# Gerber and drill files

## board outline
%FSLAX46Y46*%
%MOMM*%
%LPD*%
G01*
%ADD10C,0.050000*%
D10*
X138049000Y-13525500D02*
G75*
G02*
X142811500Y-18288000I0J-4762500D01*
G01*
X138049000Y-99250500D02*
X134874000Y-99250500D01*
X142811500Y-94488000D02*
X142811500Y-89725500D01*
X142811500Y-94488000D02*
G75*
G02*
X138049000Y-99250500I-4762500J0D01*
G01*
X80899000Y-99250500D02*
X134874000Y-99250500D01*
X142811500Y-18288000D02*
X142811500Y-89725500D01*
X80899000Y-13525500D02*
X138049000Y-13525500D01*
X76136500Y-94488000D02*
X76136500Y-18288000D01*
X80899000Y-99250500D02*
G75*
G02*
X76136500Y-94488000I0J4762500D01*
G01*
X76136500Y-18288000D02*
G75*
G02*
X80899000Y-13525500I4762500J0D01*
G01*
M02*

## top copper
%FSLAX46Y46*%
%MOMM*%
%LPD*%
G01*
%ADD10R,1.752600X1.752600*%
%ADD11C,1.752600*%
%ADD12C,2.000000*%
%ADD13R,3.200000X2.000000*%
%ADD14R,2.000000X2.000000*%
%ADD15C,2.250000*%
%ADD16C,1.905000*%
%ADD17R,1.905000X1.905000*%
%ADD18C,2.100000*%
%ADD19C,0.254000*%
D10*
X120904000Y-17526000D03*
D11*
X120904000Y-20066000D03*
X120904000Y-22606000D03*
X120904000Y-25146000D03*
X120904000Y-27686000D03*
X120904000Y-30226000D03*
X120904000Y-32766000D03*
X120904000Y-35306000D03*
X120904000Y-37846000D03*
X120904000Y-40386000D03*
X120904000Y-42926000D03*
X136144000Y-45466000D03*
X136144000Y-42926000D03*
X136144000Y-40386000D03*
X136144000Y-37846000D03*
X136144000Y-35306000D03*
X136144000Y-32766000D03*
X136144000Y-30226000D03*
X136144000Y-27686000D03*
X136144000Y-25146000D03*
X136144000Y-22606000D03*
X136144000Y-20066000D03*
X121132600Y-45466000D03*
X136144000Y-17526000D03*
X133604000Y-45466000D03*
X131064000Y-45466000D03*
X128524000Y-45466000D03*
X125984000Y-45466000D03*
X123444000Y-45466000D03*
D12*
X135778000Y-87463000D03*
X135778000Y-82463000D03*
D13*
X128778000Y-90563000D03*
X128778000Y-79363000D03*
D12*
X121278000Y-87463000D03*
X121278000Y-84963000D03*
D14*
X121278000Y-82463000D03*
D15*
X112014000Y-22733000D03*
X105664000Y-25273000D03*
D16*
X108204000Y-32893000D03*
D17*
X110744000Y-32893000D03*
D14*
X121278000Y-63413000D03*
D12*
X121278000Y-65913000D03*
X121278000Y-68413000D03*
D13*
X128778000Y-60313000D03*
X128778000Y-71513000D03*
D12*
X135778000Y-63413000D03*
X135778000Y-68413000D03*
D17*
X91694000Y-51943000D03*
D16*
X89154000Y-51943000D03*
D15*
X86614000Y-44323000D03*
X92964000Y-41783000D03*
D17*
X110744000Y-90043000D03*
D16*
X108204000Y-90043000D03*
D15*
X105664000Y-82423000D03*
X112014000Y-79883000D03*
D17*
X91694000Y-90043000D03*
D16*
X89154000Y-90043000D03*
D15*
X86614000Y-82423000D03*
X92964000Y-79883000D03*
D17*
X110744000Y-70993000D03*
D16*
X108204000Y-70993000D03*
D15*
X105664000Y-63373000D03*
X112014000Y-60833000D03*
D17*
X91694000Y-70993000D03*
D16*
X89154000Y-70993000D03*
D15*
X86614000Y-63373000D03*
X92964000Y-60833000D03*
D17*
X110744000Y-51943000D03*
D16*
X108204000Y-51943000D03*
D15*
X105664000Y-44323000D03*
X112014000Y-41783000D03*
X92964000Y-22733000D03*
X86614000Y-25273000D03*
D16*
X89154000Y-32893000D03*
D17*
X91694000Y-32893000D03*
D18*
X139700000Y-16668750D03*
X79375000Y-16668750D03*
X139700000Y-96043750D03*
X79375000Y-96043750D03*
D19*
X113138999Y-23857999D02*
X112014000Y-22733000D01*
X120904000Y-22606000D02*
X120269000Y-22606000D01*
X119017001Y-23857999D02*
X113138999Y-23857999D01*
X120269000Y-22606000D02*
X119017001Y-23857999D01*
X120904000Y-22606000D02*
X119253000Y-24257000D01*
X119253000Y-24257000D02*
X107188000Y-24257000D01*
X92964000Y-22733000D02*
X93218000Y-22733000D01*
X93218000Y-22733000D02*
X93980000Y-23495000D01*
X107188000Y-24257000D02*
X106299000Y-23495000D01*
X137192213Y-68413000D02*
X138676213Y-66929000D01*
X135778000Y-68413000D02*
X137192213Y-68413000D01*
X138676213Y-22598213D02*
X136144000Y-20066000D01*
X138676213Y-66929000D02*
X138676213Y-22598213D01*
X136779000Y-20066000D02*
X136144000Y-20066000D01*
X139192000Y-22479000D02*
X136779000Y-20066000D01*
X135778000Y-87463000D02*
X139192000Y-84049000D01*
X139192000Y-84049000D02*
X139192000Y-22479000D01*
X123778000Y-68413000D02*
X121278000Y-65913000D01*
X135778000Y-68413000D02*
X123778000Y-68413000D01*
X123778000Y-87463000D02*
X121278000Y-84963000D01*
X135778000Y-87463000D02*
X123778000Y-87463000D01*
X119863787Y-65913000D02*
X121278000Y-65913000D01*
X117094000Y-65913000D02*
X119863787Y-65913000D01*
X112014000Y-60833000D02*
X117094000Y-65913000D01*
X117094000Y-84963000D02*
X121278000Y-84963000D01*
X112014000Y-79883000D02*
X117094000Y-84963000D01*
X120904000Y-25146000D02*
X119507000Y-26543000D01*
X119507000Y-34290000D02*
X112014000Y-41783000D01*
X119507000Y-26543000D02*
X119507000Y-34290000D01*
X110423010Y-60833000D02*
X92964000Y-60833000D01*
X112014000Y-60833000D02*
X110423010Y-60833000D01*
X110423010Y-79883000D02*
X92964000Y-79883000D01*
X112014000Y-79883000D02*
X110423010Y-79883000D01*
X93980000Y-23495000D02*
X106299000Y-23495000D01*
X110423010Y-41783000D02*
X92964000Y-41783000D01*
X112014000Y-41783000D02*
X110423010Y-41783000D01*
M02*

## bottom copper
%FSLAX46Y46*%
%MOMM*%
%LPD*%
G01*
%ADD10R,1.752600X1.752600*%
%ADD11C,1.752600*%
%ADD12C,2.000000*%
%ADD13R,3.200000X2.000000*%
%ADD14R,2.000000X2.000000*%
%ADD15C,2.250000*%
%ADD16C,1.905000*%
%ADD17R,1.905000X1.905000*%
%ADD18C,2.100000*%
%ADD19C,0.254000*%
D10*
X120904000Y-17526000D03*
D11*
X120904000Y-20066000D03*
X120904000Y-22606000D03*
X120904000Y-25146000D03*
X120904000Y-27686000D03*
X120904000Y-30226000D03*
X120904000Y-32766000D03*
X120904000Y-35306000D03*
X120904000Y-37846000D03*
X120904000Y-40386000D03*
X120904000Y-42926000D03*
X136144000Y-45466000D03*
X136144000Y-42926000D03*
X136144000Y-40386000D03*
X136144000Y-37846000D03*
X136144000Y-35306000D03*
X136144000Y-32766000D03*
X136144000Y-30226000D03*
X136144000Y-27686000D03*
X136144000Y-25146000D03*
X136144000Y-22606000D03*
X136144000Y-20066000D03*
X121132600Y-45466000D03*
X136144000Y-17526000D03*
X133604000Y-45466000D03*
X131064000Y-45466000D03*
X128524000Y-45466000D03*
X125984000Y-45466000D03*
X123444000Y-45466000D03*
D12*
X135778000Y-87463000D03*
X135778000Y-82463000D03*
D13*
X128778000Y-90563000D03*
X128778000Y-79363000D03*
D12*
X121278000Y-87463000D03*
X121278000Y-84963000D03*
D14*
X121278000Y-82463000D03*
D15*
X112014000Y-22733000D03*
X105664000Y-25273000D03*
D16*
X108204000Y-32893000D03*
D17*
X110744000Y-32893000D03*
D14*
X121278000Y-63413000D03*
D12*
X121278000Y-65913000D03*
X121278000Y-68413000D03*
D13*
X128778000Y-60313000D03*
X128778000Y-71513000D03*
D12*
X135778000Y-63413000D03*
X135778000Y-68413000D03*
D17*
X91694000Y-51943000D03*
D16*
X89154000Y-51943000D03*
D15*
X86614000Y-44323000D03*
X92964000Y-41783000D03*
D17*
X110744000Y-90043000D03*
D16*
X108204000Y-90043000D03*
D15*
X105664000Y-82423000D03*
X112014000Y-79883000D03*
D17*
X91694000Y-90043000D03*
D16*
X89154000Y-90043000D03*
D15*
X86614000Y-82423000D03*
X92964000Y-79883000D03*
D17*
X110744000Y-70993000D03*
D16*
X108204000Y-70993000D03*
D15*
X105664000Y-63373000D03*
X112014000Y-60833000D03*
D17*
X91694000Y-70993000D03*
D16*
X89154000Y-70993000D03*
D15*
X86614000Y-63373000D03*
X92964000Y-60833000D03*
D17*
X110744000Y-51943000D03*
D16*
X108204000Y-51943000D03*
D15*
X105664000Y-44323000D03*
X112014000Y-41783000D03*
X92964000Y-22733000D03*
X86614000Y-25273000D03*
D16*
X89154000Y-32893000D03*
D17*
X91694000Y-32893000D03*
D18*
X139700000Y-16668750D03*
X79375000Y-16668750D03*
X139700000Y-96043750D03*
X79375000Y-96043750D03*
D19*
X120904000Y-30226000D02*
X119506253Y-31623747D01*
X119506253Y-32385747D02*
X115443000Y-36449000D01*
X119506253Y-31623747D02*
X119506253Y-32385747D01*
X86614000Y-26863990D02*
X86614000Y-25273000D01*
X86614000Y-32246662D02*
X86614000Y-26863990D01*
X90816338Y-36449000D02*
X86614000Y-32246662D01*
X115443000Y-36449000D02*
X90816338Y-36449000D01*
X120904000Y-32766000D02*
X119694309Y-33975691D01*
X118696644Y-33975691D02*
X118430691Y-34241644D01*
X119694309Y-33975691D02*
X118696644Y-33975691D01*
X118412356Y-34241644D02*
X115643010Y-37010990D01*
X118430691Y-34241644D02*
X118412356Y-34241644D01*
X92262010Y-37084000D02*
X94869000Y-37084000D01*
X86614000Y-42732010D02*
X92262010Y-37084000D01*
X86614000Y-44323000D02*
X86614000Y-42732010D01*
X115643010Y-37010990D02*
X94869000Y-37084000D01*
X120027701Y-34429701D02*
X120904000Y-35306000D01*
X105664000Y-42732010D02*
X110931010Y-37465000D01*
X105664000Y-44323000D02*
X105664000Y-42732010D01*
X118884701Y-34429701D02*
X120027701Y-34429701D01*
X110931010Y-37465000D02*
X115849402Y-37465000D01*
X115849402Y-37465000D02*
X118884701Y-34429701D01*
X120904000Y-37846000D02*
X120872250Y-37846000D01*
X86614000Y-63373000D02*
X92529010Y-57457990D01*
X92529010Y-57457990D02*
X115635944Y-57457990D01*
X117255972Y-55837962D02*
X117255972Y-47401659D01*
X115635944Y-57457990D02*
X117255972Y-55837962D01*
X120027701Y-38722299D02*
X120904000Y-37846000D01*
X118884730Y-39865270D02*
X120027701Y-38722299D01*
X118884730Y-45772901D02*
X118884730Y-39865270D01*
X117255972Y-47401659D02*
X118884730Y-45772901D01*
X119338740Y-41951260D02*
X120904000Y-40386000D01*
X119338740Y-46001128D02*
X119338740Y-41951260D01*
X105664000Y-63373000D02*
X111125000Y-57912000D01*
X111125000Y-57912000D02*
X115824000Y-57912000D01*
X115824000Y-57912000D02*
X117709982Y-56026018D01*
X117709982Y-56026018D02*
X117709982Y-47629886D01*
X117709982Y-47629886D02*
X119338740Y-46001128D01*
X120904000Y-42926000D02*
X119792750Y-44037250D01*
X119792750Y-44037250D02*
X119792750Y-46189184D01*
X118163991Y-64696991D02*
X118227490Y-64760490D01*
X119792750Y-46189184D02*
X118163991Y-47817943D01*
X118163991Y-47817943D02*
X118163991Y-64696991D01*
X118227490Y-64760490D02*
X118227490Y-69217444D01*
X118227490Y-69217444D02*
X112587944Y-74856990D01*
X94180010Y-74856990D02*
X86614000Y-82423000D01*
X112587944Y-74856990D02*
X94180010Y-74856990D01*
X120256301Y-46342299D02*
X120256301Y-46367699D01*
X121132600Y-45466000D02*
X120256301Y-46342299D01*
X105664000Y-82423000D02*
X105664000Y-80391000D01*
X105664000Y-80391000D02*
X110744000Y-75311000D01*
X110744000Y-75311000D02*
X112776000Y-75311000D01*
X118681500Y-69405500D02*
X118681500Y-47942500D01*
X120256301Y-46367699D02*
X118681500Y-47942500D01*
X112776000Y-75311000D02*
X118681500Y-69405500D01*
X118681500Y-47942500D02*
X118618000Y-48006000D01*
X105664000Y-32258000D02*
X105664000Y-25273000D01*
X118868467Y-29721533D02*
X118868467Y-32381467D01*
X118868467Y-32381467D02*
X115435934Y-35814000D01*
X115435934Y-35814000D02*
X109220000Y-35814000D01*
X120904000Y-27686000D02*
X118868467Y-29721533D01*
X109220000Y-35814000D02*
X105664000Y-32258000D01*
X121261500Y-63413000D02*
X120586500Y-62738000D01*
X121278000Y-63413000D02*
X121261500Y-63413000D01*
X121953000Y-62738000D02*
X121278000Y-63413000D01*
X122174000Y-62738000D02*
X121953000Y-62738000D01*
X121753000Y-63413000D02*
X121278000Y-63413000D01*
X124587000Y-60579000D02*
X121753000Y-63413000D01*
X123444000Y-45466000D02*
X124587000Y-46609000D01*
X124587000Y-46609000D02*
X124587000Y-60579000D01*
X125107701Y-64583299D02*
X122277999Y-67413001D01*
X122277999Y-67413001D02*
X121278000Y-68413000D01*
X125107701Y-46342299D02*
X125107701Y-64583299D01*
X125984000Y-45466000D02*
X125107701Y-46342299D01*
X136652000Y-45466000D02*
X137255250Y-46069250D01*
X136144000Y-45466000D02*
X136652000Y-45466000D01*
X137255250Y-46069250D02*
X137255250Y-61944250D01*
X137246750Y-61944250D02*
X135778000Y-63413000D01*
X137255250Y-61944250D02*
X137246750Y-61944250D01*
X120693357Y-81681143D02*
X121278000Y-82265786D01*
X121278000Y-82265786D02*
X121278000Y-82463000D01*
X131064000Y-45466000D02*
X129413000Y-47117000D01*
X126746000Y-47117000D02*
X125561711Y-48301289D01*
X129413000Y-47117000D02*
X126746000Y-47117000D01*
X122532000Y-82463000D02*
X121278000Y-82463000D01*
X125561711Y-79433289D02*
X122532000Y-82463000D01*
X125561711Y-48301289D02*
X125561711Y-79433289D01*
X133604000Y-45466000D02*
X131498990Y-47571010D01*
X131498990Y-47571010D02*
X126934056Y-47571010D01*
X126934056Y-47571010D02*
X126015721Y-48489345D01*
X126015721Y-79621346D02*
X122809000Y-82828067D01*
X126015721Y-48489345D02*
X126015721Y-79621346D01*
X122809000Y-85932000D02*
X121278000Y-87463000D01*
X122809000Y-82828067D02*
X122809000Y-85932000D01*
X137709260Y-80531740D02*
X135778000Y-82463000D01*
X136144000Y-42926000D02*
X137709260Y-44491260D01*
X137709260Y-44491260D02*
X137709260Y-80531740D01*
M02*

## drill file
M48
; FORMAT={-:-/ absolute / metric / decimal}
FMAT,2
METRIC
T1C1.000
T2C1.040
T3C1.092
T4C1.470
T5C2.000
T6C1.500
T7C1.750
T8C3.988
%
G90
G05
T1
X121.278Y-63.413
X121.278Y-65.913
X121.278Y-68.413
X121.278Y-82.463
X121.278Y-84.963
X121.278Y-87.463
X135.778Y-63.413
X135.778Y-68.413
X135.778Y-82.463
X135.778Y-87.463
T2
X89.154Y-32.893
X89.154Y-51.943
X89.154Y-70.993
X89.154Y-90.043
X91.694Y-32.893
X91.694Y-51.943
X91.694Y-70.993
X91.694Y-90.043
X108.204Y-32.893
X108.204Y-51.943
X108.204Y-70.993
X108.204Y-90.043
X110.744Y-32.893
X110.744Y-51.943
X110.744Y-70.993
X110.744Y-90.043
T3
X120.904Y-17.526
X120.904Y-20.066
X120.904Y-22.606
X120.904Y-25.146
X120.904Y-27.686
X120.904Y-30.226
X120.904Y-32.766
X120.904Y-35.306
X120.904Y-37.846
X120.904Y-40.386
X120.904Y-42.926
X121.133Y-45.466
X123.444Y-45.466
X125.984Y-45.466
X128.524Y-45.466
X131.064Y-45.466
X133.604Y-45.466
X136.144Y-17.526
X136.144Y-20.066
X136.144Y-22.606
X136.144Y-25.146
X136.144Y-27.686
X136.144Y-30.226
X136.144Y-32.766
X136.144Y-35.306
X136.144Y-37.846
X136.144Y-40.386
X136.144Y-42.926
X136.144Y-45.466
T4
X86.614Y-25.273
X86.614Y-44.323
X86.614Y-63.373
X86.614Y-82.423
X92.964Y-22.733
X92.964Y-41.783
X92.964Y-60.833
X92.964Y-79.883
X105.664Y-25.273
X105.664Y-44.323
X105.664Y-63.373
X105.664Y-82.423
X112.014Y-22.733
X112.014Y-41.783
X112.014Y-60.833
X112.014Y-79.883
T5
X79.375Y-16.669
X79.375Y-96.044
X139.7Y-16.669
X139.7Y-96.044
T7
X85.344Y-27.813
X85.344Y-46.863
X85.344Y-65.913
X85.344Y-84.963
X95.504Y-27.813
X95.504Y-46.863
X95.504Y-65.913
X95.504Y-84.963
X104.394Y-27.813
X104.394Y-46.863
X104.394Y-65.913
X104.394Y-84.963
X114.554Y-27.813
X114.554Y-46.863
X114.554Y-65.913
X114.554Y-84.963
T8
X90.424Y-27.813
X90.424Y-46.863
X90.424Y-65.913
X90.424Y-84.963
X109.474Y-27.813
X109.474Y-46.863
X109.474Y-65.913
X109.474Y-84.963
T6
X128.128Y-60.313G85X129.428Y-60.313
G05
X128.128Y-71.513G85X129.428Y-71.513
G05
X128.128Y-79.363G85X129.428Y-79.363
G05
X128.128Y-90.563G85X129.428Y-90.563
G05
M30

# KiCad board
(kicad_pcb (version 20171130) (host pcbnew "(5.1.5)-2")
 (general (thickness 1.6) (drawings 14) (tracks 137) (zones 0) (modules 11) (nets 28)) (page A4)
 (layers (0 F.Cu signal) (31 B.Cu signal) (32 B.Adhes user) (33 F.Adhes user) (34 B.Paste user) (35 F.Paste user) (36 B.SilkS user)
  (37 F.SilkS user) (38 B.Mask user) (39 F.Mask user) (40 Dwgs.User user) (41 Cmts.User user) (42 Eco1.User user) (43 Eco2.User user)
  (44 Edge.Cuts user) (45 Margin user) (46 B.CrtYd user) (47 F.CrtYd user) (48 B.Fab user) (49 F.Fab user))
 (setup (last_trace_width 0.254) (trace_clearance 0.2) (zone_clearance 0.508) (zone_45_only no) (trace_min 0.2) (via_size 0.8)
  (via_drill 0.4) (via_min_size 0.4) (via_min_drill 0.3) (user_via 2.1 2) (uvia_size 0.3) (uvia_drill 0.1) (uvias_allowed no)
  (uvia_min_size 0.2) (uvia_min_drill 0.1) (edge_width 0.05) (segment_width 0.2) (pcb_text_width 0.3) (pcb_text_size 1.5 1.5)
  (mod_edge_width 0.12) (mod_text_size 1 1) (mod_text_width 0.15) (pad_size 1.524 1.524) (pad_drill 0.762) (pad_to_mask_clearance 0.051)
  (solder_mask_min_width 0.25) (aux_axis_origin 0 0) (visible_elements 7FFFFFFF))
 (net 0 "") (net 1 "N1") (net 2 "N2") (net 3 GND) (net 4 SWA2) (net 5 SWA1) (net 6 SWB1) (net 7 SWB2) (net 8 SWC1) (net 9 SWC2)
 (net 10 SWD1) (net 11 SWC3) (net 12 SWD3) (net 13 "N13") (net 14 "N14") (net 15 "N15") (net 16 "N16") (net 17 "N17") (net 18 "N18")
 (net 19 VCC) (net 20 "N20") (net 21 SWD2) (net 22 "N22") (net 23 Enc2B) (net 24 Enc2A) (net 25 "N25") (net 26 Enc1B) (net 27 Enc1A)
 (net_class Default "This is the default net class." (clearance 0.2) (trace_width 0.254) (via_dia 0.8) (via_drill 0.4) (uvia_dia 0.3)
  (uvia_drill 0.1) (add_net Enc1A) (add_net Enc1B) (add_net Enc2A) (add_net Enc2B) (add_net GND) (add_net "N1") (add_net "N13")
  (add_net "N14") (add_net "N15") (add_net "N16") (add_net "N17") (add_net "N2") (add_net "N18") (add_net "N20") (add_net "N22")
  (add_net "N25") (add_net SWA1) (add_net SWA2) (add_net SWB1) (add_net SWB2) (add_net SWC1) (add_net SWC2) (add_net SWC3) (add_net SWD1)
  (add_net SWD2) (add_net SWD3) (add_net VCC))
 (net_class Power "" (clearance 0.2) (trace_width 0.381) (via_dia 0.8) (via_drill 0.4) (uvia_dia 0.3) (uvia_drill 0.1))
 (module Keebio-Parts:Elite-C (layer F.Cu) (at 128.524 31.496 270)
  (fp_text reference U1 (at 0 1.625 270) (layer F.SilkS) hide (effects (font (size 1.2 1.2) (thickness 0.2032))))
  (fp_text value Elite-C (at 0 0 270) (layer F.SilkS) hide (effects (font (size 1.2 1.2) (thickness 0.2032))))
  (pad 1 thru_hole rect (at -13.97 7.62 270) (size 1.7526 1.7526) (drill 1.0922) (layers *.Cu *.SilkS *.Mask) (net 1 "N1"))
  (pad 2 thru_hole circle (at -11.43 7.62 270) (size 1.7526 1.7526) (drill 1.0922) (layers *.Cu *.SilkS *.Mask) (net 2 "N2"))
  (pad 3 thru_hole circle (at -8.89 7.62 270) (size 1.7526 1.7526) (drill 1.0922) (layers *.Cu *.SilkS *.Mask) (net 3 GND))
  (pad 4 thru_hole circle (at -6.35 7.62 270) (size 1.7526 1.7526) (drill 1.0922) (layers *.Cu *.SilkS *.Mask) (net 3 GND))
  (pad 5 thru_hole circle (at -3.81 7.62 270) (size 1.7526 1.7526) (drill 1.0922) (layers *.Cu *.SilkS *.Mask) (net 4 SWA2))
  (pad 6 thru_hole circle (at -1.27 7.62 270) (size 1.7526 1.7526) (drill 1.0922) (layers *.Cu *.SilkS *.Mask) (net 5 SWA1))
  (pad 7 thru_hole circle (at 1.27 7.62 270) (size 1.7526 1.7526) (drill 1.0922) (layers *.Cu *.SilkS *.Mask) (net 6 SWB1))
  (pad 8 thru_hole circle (at 3.81 7.62 270) (size 1.7526 1.7526) (drill 1.0922) (layers *.Cu *.SilkS *.Mask) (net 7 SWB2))
  (pad 9 thru_hole circle (at 6.35 7.62 270) (size 1.7526 1.7526) (drill 1.0922) (layers *.Cu *.SilkS *.Mask) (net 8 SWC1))
  (pad 10 thru_hole circle (at 8.89 7.62 270) (size 1.7526 1.7526) (drill 1.0922) (layers *.Cu *.SilkS *.Mask) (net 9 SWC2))
  (pad 11 thru_hole circle (at 11.43 7.62 270) (size 1.7526 1.7526) (drill 1.0922) (layers *.Cu *.SilkS *.Mask) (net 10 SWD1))
  (pad 13 thru_hole circle (at 13.97 -7.62 270) (size 1.7526 1.7526) (drill 1.0922) (layers *.Cu *.SilkS *.Mask) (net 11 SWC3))
  (pad 14 thru_hole circle (at 11.43 -7.62 270) (size 1.7526 1.7526) (drill 1.0922) (layers *.Cu *.SilkS *.Mask) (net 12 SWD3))
  (pad 15 thru_hole circle (at 8.89 -7.62 270) (size 1.7526 1.7526) (drill 1.0922) (layers *.Cu *.SilkS *.Mask) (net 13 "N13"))
  (pad 16 thru_hole circle (at 6.35 -7.62 270) (size 1.7526 1.7526) (drill 1.0922) (layers *.Cu *.SilkS *.Mask) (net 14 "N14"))
  (pad 17 thru_hole circle (at 3.81 -7.62 270) (size 1.7526 1.7526) (drill 1.0922) (layers *.Cu *.SilkS *.Mask) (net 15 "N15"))
  (pad 18 thru_hole circle (at 1.27 -7.62 270) (size 1.7526 1.7526) (drill 1.0922) (layers *.Cu *.SilkS *.Mask) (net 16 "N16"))
  (pad 19 thru_hole circle (at -1.27 -7.62 270) (size 1.7526 1.7526) (drill 1.0922) (layers *.Cu *.SilkS *.Mask) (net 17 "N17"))
  (pad 20 thru_hole circle (at -3.81 -7.62 270) (size 1.7526 1.7526) (drill 1.0922) (layers *.Cu *.SilkS *.Mask) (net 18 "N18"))
  (pad 21 thru_hole circle (at -6.35 -7.62 270) (size 1.7526 1.7526) (drill 1.0922) (layers *.Cu *.SilkS *.Mask) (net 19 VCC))
  (pad 22 thru_hole circle (at -8.89 -7.62 270) (size 1.7526 1.7526) (drill 1.0922) (layers *.Cu *.SilkS *.Mask) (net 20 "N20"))
  (pad 23 thru_hole circle (at -11.43 -7.62 270) (size 1.7526 1.7526) (drill 1.0922) (layers *.Cu *.SilkS *.Mask) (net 3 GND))
  (pad 12 thru_hole circle (at 13.97 7.3914 270) (size 1.7526 1.7526) (drill 1.0922) (layers *.Cu *.SilkS *.Mask) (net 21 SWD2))
  (pad 24 thru_hole circle (at -13.97 -7.62 270) (size 1.7526 1.7526) (drill 1.0922) (layers *.Cu *.SilkS *.Mask) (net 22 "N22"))
  (pad 29 thru_hole circle (at 13.97 -5.08 270) (size 1.7526 1.7526) (drill 1.0922) (layers *.Cu *.SilkS *.Mask) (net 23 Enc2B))
  (pad 28 thru_hole circle (at 13.97 -2.54 270) (size 1.7526 1.7526) (drill 1.0922) (layers *.Cu *.SilkS *.Mask) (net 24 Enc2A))
  (pad 27 thru_hole circle (at 13.97 0 270) (size 1.7526 1.7526) (drill 1.0922) (layers *.Cu *.SilkS *.Mask) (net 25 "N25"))
  (pad 26 thru_hole circle (at 13.97 2.54 270) (size 1.7526 1.7526) (drill 1.0922) (layers *.Cu *.SilkS *.Mask) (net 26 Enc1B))
  (pad 25 thru_hole circle (at 13.97 5.08 270) (size 1.7526 1.7526) (drill 1.0922) (layers *.Cu *.SilkS *.Mask) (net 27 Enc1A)))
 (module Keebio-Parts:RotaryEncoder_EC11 (layer F.Cu) (at 128.778 84.963)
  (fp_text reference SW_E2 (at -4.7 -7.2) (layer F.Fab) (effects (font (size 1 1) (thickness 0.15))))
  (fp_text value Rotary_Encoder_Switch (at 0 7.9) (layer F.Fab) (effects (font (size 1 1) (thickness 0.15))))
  (pad S1 thru_hole circle (at 7 2.5) (size 2 2) (drill 1) (layers *.Cu *.Mask) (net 3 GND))
  (pad S2 thru_hole circle (at 7 -2.5) (size 2 2) (drill 1) (layers *.Cu *.Mask) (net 12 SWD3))
  (pad "" np_thru_hole rect (at 0 5.6) (size 3.2 2) (drill oval 2.8 1.5) (layers *.Cu *.Mask))
  (pad "" np_thru_hole rect (at 0 -5.6) (size 3.2 2) (drill oval 2.8 1.5) (layers *.Cu *.Mask))
  (pad B thru_hole circle (at -7.5 2.5) (size 2 2) (drill 1) (layers *.Cu *.Mask) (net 23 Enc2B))
  (pad C thru_hole circle (at -7.5 0) (size 2 2) (drill 1) (layers *.Cu *.Mask) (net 3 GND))
  (pad A thru_hole rect (at -7.5 -2.5) (size 2 2) (drill 1) (layers *.Cu *.Mask) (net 24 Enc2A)))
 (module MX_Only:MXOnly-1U (layer F.Cu) (at 109.474 27.813)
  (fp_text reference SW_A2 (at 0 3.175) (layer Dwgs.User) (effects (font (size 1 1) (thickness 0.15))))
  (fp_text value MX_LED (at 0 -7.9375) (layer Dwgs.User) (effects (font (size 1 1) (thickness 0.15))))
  (pad 2 thru_hole circle (at 2.54 -5.08) (size 2.25 2.25) (drill 1.47) (layers *.Cu B.Mask) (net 3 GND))
  (pad "" np_thru_hole circle (at 0 0) (size 3.9878 3.9878) (drill 3.9878) (layers *.Cu *.Mask))
  (pad 1 thru_hole circle (at -3.81 -2.54) (size 2.25 2.25) (drill 1.47) (layers *.Cu B.Mask) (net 4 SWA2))
  (pad 3 thru_hole circle (at -1.27 5.08) (size 1.905 1.905) (drill 1.04) (layers *.Cu B.Mask))
  (pad 4 thru_hole rect (at 1.27 5.08) (size 1.905 1.905) (drill 1.04) (layers *.Cu B.Mask))
  (pad "" np_thru_hole circle (at -5.08 0 48.0996) (size 1.75 1.75) (drill 1.75) (layers *.Cu *.Mask))
  (pad "" np_thru_hole circle (at 5.08 0 48.0996) (size 1.75 1.75) (drill 1.75) (layers *.Cu *.Mask)))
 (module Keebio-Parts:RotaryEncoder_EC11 (layer F.Cu) (at 128.778 65.913)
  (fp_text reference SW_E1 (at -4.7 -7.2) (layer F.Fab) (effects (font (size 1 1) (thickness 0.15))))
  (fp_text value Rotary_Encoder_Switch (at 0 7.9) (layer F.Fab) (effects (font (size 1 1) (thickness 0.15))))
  (pad A thru_hole rect (at -7.5 -2.5) (size 2 2) (drill 1) (layers *.Cu *.Mask) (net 27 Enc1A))
  (pad C thru_hole circle (at -7.5 0) (size 2 2) (drill 1) (layers *.Cu *.Mask) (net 3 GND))
  (pad B thru_hole circle (at -7.5 2.5) (size 2 2) (drill 1) (layers *.Cu *.Mask) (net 26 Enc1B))
  (pad "" np_thru_hole rect (at 0 -5.6) (size 3.2 2) (drill oval 2.8 1.5) (layers *.Cu *.Mask))
  (pad "" np_thru_hole rect (at 0 5.6) (size 3.2 2) (drill oval 2.8 1.5) (layers *.Cu *.Mask))
  (pad S2 thru_hole circle (at 7 -2.5) (size 2 2) (drill 1) (layers *.Cu *.Mask) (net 11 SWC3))
  (pad S1 thru_hole circle (at 7 2.5) (size 2 2) (drill 1) (layers *.Cu *.Mask) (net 3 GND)))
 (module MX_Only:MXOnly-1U (layer F.Cu) (at 90.424 46.863)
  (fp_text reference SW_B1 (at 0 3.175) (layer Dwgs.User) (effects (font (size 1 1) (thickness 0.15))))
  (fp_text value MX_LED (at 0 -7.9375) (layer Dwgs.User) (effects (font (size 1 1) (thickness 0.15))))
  (pad "" np_thru_hole circle (at 5.08 0 48.0996) (size 1.75 1.75) (drill 1.75) (layers *.Cu *.Mask))
  (pad "" np_thru_hole circle (at -5.08 0 48.0996) (size 1.75 1.75) (drill 1.75) (layers *.Cu *.Mask))
  (pad 4 thru_hole rect (at 1.27 5.08) (size 1.905 1.905) (drill 1.04) (layers *.Cu B.Mask))
  (pad 3 thru_hole circle (at -1.27 5.08) (size 1.905 1.905) (drill 1.04) (layers *.Cu B.Mask))
  (pad 1 thru_hole circle (at -3.81 -2.54) (size 2.25 2.25) (drill 1.47) (layers *.Cu B.Mask) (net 6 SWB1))
  (pad "" np_thru_hole circle (at 0 0) (size 3.9878 3.9878) (drill 3.9878) (layers *.Cu *.Mask))
  (pad 2 thru_hole circle (at 2.54 -5.08) (size 2.25 2.25) (drill 1.47) (layers *.Cu B.Mask) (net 3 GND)))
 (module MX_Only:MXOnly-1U (layer F.Cu) (at 109.474 84.963)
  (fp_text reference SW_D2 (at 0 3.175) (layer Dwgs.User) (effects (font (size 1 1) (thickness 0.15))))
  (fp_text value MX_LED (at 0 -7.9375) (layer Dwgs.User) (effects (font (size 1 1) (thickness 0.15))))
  (pad "" np_thru_hole circle (at 5.08 0 48.0996) (size 1.75 1.75) (drill 1.75) (layers *.Cu *.Mask))
  (pad "" np_thru_hole circle (at -5.08 0 48.0996) (size 1.75 1.75) (drill 1.75) (layers *.Cu *.Mask))
  (pad 4 thru_hole rect (at 1.27 5.08) (size 1.905 1.905) (drill 1.04) (layers *.Cu B.Mask))
  (pad 3 thru_hole circle (at -1.27 5.08) (size 1.905 1.905) (drill 1.04) (layers *.Cu B.Mask))
  (pad 1 thru_hole circle (at -3.81 -2.54) (size 2.25 2.25) (drill 1.47) (layers *.Cu B.Mask) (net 21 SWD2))
  (pad "" np_thru_hole circle (at 0 0) (size 3.9878 3.9878) (drill 3.9878) (layers *.Cu *.Mask))
  (pad 2 thru_hole circle (at 2.54 -5.08) (size 2.25 2.25) (drill 1.47) (layers *.Cu B.Mask) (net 3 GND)))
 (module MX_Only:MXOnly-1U (layer F.Cu) (at 90.424 84.963)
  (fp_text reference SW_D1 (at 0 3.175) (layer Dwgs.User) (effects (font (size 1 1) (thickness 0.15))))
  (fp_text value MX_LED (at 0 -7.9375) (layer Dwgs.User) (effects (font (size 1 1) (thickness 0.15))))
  (pad "" np_thru_hole circle (at 5.08 0 48.0996) (size 1.75 1.75) (drill 1.75) (layers *.Cu *.Mask))
  (pad "" np_thru_hole circle (at -5.08 0 48.0996) (size 1.75 1.75) (drill 1.75) (layers *.Cu *.Mask))
  (pad 4 thru_hole rect (at 1.27 5.08) (size 1.905 1.905) (drill 1.04) (layers *.Cu B.Mask))
  (pad 3 thru_hole circle (at -1.27 5.08) (size 1.905 1.905) (drill 1.04) (layers *.Cu B.Mask))
  (pad 1 thru_hole circle (at -3.81 -2.54) (size 2.25 2.25) (drill 1.47) (layers *.Cu B.Mask) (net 10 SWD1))
  (pad "" np_thru_hole circle (at 0 0) (size 3.9878 3.9878) (drill 3.9878) (layers *.Cu *.Mask))
  (pad 2 thru_hole circle (at 2.54 -5.08) (size 2.25 2.25) (drill 1.47) (layers *.Cu B.Mask) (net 3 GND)))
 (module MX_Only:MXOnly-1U (layer F.Cu) (at 109.474 65.913)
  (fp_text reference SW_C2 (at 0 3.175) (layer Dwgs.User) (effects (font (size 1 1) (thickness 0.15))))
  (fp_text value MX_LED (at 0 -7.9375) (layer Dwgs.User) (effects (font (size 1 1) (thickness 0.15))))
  (pad "" np_thru_hole circle (at 5.08 0 48.0996) (size 1.75 1.75) (drill 1.75) (layers *.Cu *.Mask))
  (pad "" np_thru_hole circle (at -5.08 0 48.0996) (size 1.75 1.75) (drill 1.75) (layers *.Cu *.Mask))
  (pad 4 thru_hole rect (at 1.27 5.08) (size 1.905 1.905) (drill 1.04) (layers *.Cu B.Mask))
  (pad 3 thru_hole circle (at -1.27 5.08) (size 1.905 1.905) (drill 1.04) (layers *.Cu B.Mask))
  (pad 1 thru_hole circle (at -3.81 -2.54) (size 2.25 2.25) (drill 1.47) (layers *.Cu B.Mask) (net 9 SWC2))
  (pad "" np_thru_hole circle (at 0 0) (size 3.9878 3.9878) (drill 3.9878) (layers *.Cu *.Mask))
  (pad 2 thru_hole circle (at 2.54 -5.08) (size 2.25 2.25) (drill 1.47) (layers *.Cu B.Mask) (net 3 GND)))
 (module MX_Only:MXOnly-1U (layer F.Cu) (at 90.424 65.913)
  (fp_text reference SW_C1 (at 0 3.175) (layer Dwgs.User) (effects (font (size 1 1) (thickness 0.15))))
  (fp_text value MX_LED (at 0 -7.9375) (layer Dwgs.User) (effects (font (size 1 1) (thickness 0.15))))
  (pad "" np_thru_hole circle (at 5.08 0 48.0996) (size 1.75 1.75) (drill 1.75) (layers *.Cu *.Mask))
  (pad "" np_thru_hole circle (at -5.08 0 48.0996) (size 1.75 1.75) (drill 1.75) (layers *.Cu *.Mask))
  (pad 4 thru_hole rect (at 1.27 5.08) (size 1.905 1.905) (drill 1.04) (layers *.Cu B.Mask))
  (pad 3 thru_hole circle (at -1.27 5.08) (size 1.905 1.905) (drill 1.04) (layers *.Cu B.Mask))
  (pad 1 thru_hole circle (at -3.81 -2.54) (size 2.25 2.25) (drill 1.47) (layers *.Cu B.Mask) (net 8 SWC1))
  (pad "" np_thru_hole circle (at 0 0) (size 3.9878 3.9878) (drill 3.9878) (layers *.Cu *.Mask))
  (pad 2 thru_hole circle (at 2.54 -5.08) (size 2.25 2.25) (drill 1.47) (layers *.Cu B.Mask) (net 3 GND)))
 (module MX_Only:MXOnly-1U (layer F.Cu) (at 109.474 46.863)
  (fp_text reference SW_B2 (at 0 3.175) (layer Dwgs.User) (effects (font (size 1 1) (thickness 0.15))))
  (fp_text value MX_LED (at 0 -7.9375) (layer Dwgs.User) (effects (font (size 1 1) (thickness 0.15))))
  (pad "" np_thru_hole circle (at 5.08 0 48.0996) (size 1.75 1.75) (drill 1.75) (layers *.Cu *.Mask))
  (pad "" np_thru_hole circle (at -5.08 0 48.0996) (size 1.75 1.75) (drill 1.75) (layers *.Cu *.Mask))
  (pad 4 thru_hole rect (at 1.27 5.08) (size 1.905 1.905) (drill 1.04) (layers *.Cu B.Mask))
  (pad 3 thru_hole circle (at -1.27 5.08) (size 1.905 1.905) (drill 1.04) (layers *.Cu B.Mask))
  (pad 1 thru_hole circle (at -3.81 -2.54) (size 2.25 2.25) (drill 1.47) (layers *.Cu B.Mask) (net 7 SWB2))
  (pad "" np_thru_hole circle (at 0 0) (size 3.9878 3.9878) (drill 3.9878) (layers *.Cu *.Mask))
  (pad 2 thru_hole circle (at 2.54 -5.08) (size 2.25 2.25) (drill 1.47) (layers *.Cu B.Mask) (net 3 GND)))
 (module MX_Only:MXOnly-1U (layer F.Cu) (at 90.424 27.813)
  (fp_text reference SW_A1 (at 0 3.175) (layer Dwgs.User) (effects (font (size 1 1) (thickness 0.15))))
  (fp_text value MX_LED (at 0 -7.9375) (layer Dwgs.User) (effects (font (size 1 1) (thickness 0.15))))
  (pad 2 thru_hole circle (at 2.54 -5.08) (size 2.25 2.25) (drill 1.47) (layers *.Cu B.Mask) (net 3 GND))
  (pad "" np_thru_hole circle (at 0 0) (size 3.9878 3.9878) (drill 3.9878) (layers *.Cu *.Mask))
  (pad 1 thru_hole circle (at -3.81 -2.54) (size 2.25 2.25) (drill 1.47) (layers *.Cu B.Mask) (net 5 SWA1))
  (pad 3 thru_hole circle (at -1.27 5.08) (size 1.905 1.905) (drill 1.04) (layers *.Cu B.Mask))
  (pad 4 thru_hole rect (at 1.27 5.08) (size 1.905 1.905) (drill 1.04) (layers *.Cu B.Mask))
  (pad "" np_thru_hole circle (at -5.08 0 48.0996) (size 1.75 1.75) (drill 1.75) (layers *.Cu *.Mask))
  (pad "" np_thru_hole circle (at 5.08 0 48.0996) (size 1.75 1.75) (drill 1.75) (layers *.Cu *.Mask)))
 (gr_arc (start 138.049 18.288) (end 142.8115 18.288) (angle -90) (layer Edge.Cuts) (width 0.05))
 (gr_line (start 138.049 99.2505) (end 134.874 99.2505) (layer Edge.Cuts) (width 0.05))
 (gr_line (start 142.8115 94.488) (end 142.8115 89.7255) (layer Edge.Cuts) (width 0.05))
 (gr_arc (start 138.049 94.488) (end 138.049 99.2505) (angle -90) (layer Edge.Cuts) (width 0.05))
 (gr_line (start 80.899 99.2505) (end 134.874 99.2505) (layer Edge.Cuts) (width 0.05))
 (gr_line (start 142.8115 18.288) (end 142.8115 89.7255) (layer Edge.Cuts) (width 0.05))
 (gr_line (start 80.899 13.5255) (end 138.049 13.5255) (layer Edge.Cuts) (width 0.05))
 (gr_line (start 76.1365 94.488) (end 76.1365 18.288) (layer Edge.Cuts) (width 0.05))
 (gr_arc (start 80.899 94.488) (end 76.1365 94.488) (angle -90) (layer Edge.Cuts) (width 0.05))
 (gr_arc (start 80.899 18.288) (end 80.899 13.5255) (angle -90) (layer Edge.Cuts) (width 0.05))
 (via (at 139.7 16.66875) (size 2.1) (drill 2) (layers F.Cu B.Cu) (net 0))
 (via (at 79.375 16.66875) (size 2.1) (drill 2) (layers F.Cu B.Cu) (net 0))
 (via (at 139.7 96.04375) (size 2.1) (drill 2) (layers F.Cu B.Cu) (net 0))
 (via (at 79.375 96.04375) (size 2.1) (drill 2) (layers F.Cu B.Cu) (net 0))
 (segment (start 120.904 30.226) (end 119.506253 31.623747) (width 0.254) (layer B.Cu) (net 5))
 (segment (start 119.506253 32.385747) (end 115.443 36.449) (width 0.254) (layer B.Cu) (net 5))
 (segment (start 119.506253 31.623747) (end 119.506253 32.385747) (width 0.254) (layer B.Cu) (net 5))
 (segment (start 86.614 26.86399) (end 86.614 25.273) (width 0.254) (layer B.Cu) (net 5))
 (segment (start 86.614 32.246662) (end 86.614 26.86399) (width 0.254) (layer B.Cu) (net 5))
 (segment (start 90.816338 36.449) (end 86.614 32.246662) (width 0.254) (layer B.Cu) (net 5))
 (segment (start 115.443 36.449) (end 90.816338 36.449) (width 0.254) (layer B.Cu) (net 5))
 (segment (start 113.138999 23.857999) (end 112.014 22.733) (width 0.254) (layer F.Cu) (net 3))
 (segment (start 120.904 22.606) (end 120.269 22.606) (width 0.254) (layer F.Cu) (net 3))
 (segment (start 119.017001 23.857999) (end 113.138999 23.857999) (width 0.254) (layer F.Cu) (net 3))
 (segment (start 120.269 22.606) (end 119.017001 23.857999) (width 0.254) (layer F.Cu) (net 3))
 (segment (start 120.904 22.606) (end 119.253 24.257) (width 0.254) (layer F.Cu) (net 3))
 (segment (start 119.253 24.257) (end 107.188 24.257) (width 0.254) (layer F.Cu) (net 3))
 (segment (start 92.964 22.733) (end 93.218 22.733) (width 0.254) (layer F.Cu) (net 3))
 (segment (start 93.218 22.733) (end 93.98 23.495) (width 0.254) (layer F.Cu) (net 3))
 (segment (start 107.188 24.257) (end 106.299 23.495) (width 0.254) (layer F.Cu) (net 3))
 (segment (start 137.192213 68.413) (end 138.676213 66.929) (width 0.254) (layer F.Cu) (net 3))
 (segment (start 135.778 68.413) (end 137.192213 68.413) (width 0.254) (layer F.Cu) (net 3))
 (segment (start 138.676213 22.598213) (end 136.144 20.066) (width 0.254) (layer F.Cu) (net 3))
 (segment (start 138.676213 66.929) (end 138.676213 22.598213) (width 0.254) (layer F.Cu) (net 3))
 (segment (start 136.779 20.066) (end 136.144 20.066) (width 0.254) (layer F.Cu) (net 3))
 (segment (start 139.192 22.479) (end 136.779 20.066) (width 0.254) (layer F.Cu) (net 3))
 (segment (start 135.778 87.463) (end 139.192 84.049) (width 0.254) (layer F.Cu) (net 3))
 (segment (start 139.192 84.049) (end 139.192 22.479) (width 0.254) (layer F.Cu) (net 3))
 (segment (start 123.778 68.413) (end 121.278 65.913) (width 0.254) (layer F.Cu) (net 3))
 (segment (start 135.778 68.413) (end 123.778 68.413) (width 0.254) (layer F.Cu) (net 3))
 (segment (start 123.778 87.463) (end 121.278 84.963) (width 0.254) (layer F.Cu) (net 3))
 (segment (start 135.778 87.463) (end 123.778 87.463) (width 0.254) (layer F.Cu) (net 3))
 (segment (start 119.863787 65.913) (end 121.278 65.913) (width 0.254) (layer F.Cu) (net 3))
 (segment (start 117.094 65.913) (end 119.863787 65.913) (width 0.254) (layer F.Cu) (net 3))
 (segment (start 112.014 60.833) (end 117.094 65.913) (width 0.254) (layer F.Cu) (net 3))
 (segment (start 117.094 84.963) (end 121.278 84.963) (width 0.254) (layer F.Cu) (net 3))
 (segment (start 112.014 79.883) (end 117.094 84.963) (width 0.254) (layer F.Cu) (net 3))
 (segment (start 120.904 25.146) (end 119.507 26.543) (width 0.254) (layer F.Cu) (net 3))
 (segment (start 119.507 34.29) (end 112.014 41.783) (width 0.254) (layer F.Cu) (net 3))
 (segment (start 119.507 26.543) (end 119.507 34.29) (width 0.254) (layer F.Cu) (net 3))
 (segment (start 110.42301 60.833) (end 92.964 60.833) (width 0.254) (layer F.Cu) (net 3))
 (segment (start 112.014 60.833) (end 110.42301 60.833) (width 0.254) (layer F.Cu) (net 3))
 (segment (start 110.42301 79.883) (end 92.964 79.883) (width 0.254) (layer F.Cu) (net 3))
 (segment (start 112.014 79.883) (end 110.42301 79.883) (width 0.254) (layer F.Cu) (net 3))
 (segment (start 93.98 23.495) (end 106.299 23.495) (width 0.254) (layer F.Cu) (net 3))
 (segment (start 110.42301 41.783) (end 92.964 41.783) (width 0.254) (layer F.Cu) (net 3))
 (segment (start 112.014 41.783) (end 110.42301 41.783) (width 0.254) (layer F.Cu) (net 3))
 (segment (start 120.904 32.766) (end 119.694309 33.975691) (width 0.254) (layer B.Cu) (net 6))
 (segment (start 118.696644 33.975691) (end 118.430691 34.241644) (width 0.254) (layer B.Cu) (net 6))
 (segment (start 119.694309 33.975691) (end 118.696644 33.975691) (width 0.254) (layer B.Cu) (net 6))
 (segment (start 118.412356 34.241644) (end 115.64301 37.01099) (width 0.254) (layer B.Cu) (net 6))
 (segment (start 118.430691 34.241644) (end 118.412356 34.241644) (width 0.254) (layer B.Cu) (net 6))
 (segment (start 92.26201 37.084) (end 94.869 37.084) (width 0.254) (layer B.Cu) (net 6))
 (segment (start 86.614 42.73201) (end 92.26201 37.084) (width 0.254) (layer B.Cu) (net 6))
 (segment (start 86.614 44.323) (end 86.614 42.73201) (width 0.254) (layer B.Cu) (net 6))
 (segment (start 115.64301 37.01099) (end 94.869 37.084) (width 0.254) (layer B.Cu) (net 6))
 (segment (start 120.027701 34.429701) (end 120.904 35.306) (width 0.254) (layer B.Cu) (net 7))
 (segment (start 105.664 42.73201) (end 110.93101 37.465) (width 0.254) (layer B.Cu) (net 7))
 (segment (start 105.664 44.323) (end 105.664 42.73201) (width 0.254) (layer B.Cu) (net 7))
 (segment (start 118.884701 34.429701) (end 120.027701 34.429701) (width 0.254) (layer B.Cu) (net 7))
 (segment (start 110.93101 37.465) (end 115.849402 37.465) (width 0.254) (layer B.Cu) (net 7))
 (segment (start 115.849402 37.465) (end 118.884701 34.429701) (width 0.254) (layer B.Cu) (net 7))
 (segment (start 120.904 37.846) (end 120.87225 37.846) (width 0.254) (layer B.Cu) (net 8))
 (segment (start 86.614 63.373) (end 92.52901 57.45799) (width 0.254) (layer B.Cu) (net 8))
 (segment (start 92.52901 57.45799) (end 115.635944 57.45799) (width 0.254) (layer B.Cu) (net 8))
 (segment (start 117.255972 55.837962) (end 117.255972 47.401659) (width 0.254) (layer B.Cu) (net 8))
 (segment (start 115.635944 57.45799) (end 117.255972 55.837962) (width 0.254) (layer B.Cu) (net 8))
 (segment (start 120.027701 38.722299) (end 120.904 37.846) (width 0.254) (layer B.Cu) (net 8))
 (segment (start 118.88473 39.86527) (end 120.027701 38.722299) (width 0.254) (layer B.Cu) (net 8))
 (segment (start 118.88473 45.772901) (end 118.88473 39.86527) (width 0.254) (layer B.Cu) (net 8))
 (segment (start 117.255972 47.401659) (end 118.88473 45.772901) (width 0.254) (layer B.Cu) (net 8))
 (segment (start 119.33874 41.95126) (end 120.904 40.386) (width 0.254) (layer B.Cu) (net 9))
 (segment (start 119.33874 46.001128) (end 119.33874 41.95126) (width 0.254) (layer B.Cu) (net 9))
 (segment (start 105.664 63.373) (end 111.125 57.912) (width 0.254) (layer B.Cu) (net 9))
 (segment (start 111.125 57.912) (end 115.824 57.912) (width 0.254) (layer B.Cu) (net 9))
 (segment (start 115.824 57.912) (end 117.709982 56.026018) (width 0.254) (layer B.Cu) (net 9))
 (segment (start 117.709982 56.026018) (end 117.709982 47.629886) (width 0.254) (layer B.Cu) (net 9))
 (segment (start 117.709982 47.629886) (end 119.33874 46.001128) (width 0.254) (layer B.Cu) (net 9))
 (segment (start 120.904 42.926) (end 119.79275 44.03725) (width 0.254) (layer B.Cu) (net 10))
 (segment (start 119.79275 44.03725) (end 119.79275 46.189184) (width 0.254) (layer B.Cu) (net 10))
 (segment (start 118.163991 64.696991) (end 118.22749 64.76049) (width 0.254) (layer B.Cu) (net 10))
 (segment (start 119.79275 46.189184) (end 118.163991 47.817943) (width 0.254) (layer B.Cu) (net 10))
 (segment (start 118.163991 47.817943) (end 118.163991 64.696991) (width 0.254) (layer B.Cu) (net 10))
 (segment (start 118.22749 64.76049) (end 118.22749 69.217444) (width 0.254) (layer B.Cu) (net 10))
 (segment (start 118.22749 69.217444) (end 112.587944 74.85699) (width 0.254) (layer B.Cu) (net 10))
 (segment (start 94.18001 74.85699) (end 86.614 82.423) (width 0.254) (layer B.Cu) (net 10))
 (segment (start 112.587944 74.85699) (end 94.18001 74.85699) (width 0.254) (layer B.Cu) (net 10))
 (segment (start 120.256301 46.342299) (end 120.256301 46.367699) (width 0.254) (layer B.Cu) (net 21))
 (segment (start 121.1326 45.466) (end 120.256301 46.342299) (width 0.254) (layer B.Cu) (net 21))
 (segment (start 105.664 82.423) (end 105.664 80.391) (width 0.254) (layer B.Cu) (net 21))
 (segment (start 105.664 80.391) (end 110.744 75.311) (width 0.254) (layer B.Cu) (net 21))
 (segment (start 110.744 75.311) (end 112.776 75.311) (width 0.254) (layer B.Cu) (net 21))
 (segment (start 118.6815 69.4055) (end 118.6815 47.9425) (width 0.254) (layer B.Cu) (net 21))
 (segment (start 120.256301 46.367699) (end 118.6815 47.9425) (width 0.254) (layer B.Cu) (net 21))
 (segment (start 112.776 75.311) (end 118.6815 69.4055) (width 0.254) (layer B.Cu) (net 21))
 (segment (start 118.6815 47.9425) (end 118.618 48.006) (width 0.254) (layer B.Cu) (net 21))
 (segment (start 105.664 32.258) (end 105.664 25.273) (width 0.254) (layer B.Cu) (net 4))
 (segment (start 118.868467 29.721533) (end 118.868467 32.381467) (width 0.254) (layer B.Cu) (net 4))
 (segment (start 118.868467 32.381467) (end 115.435934 35.814) (width 0.254) (layer B.Cu) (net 4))
 (segment (start 115.435934 35.814) (end 109.22 35.814) (width 0.254) (layer B.Cu) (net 4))
 (segment (start 120.904 27.686) (end 118.868467 29.721533) (width 0.254) (layer B.Cu) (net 4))
 (segment (start 109.22 35.814) (end 105.664 32.258) (width 0.254) (layer B.Cu) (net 4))
 (segment (start 121.2615 63.413) (end 120.5865 62.738) (width 0.254) (layer B.Cu) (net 27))
 (segment (start 121.278 63.413) (end 121.2615 63.413) (width 0.254) (layer B.Cu) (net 27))
 (segment (start 121.953 62.738) (end 121.278 63.413) (width 0.254) (layer B.Cu) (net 27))
 (segment (start 122.174 62.738) (end 121.953 62.738) (width 0.254) (layer B.Cu) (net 27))
 (segment (start 121.753 63.413) (end 121.278 63.413) (width 0.254) (layer B.Cu) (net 27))
 (segment (start 124.587 60.579) (end 121.753 63.413) (width 0.254) (layer B.Cu) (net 27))
 (segment (start 123.444 45.466) (end 124.587 46.609) (width 0.254) (layer B.Cu) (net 27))
 (segment (start 124.587 46.609) (end 124.587 60.579) (width 0.254) (layer B.Cu) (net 27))
 (segment (start 125.107701 64.583299) (end 122.277999 67.413001) (width 0.254) (layer B.Cu) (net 26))
 (segment (start 122.277999 67.413001) (end 121.278 68.413) (width 0.254) (layer B.Cu) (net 26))
 (segment (start 125.107701 46.342299) (end 125.107701 64.583299) (width 0.254) (layer B.Cu) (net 26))
 (segment (start 125.984 45.466) (end 125.107701 46.342299) (width 0.254) (layer B.Cu) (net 26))
 (segment (start 136.652 45.466) (end 137.25525 46.06925) (width 0.254) (layer B.Cu) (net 11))
 (segment (start 136.144 45.466) (end 136.652 45.466) (width 0.254) (layer B.Cu) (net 11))
 (segment (start 137.25525 46.06925) (end 137.25525 61.94425) (width 0.254) (layer B.Cu) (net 11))
 (segment (start 137.24675 61.94425) (end 135.778 63.413) (width 0.254) (layer B.Cu) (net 11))
 (segment (start 137.25525 61.94425) (end 137.24675 61.94425) (width 0.254) (layer B.Cu) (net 11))
 (segment (start 120.693357 81.681143) (end 121.278 82.265786) (width 0.254) (layer B.Cu) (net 24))
 (segment (start 121.278 82.265786) (end 121.278 82.463) (width 0.254) (layer B.Cu) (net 24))
 (segment (start 131.064 45.466) (end 129.413 47.117) (width 0.254) (layer B.Cu) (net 24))
 (segment (start 126.746 47.117) (end 125.561711 48.301289) (width 0.254) (layer B.Cu) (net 24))
 (segment (start 129.413 47.117) (end 126.746 47.117) (width 0.254) (layer B.Cu) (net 24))
 (segment (start 122.532 82.463) (end 121.278 82.463) (width 0.254) (layer B.Cu) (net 24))
 (segment (start 125.561711 79.433289) (end 122.532 82.463) (width 0.254) (layer B.Cu) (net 24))
 (segment (start 125.561711 48.301289) (end 125.561711 79.433289) (width 0.254) (layer B.Cu) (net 24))
 (segment (start 133.604 45.466) (end 131.49899 47.57101) (width 0.254) (layer B.Cu) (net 23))
 (segment (start 131.49899 47.57101) (end 126.934056 47.57101) (width 0.254) (layer B.Cu) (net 23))
 (segment (start 126.934056 47.57101) (end 126.015721 48.489345) (width 0.254) (layer B.Cu) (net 23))
 (segment (start 126.015721 79.621346) (end 122.809 82.828067) (width 0.254) (layer B.Cu) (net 23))
 (segment (start 126.015721 48.489345) (end 126.015721 79.621346) (width 0.254) (layer B.Cu) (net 23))
 (segment (start 122.809 85.932) (end 121.278 87.463) (width 0.254) (layer B.Cu) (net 23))
 (segment (start 122.809 82.828067) (end 122.809 85.932) (width 0.254) (layer B.Cu) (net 23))
 (segment (start 137.70926 80.53174) (end 135.778 82.463) (width 0.254) (layer B.Cu) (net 12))
 (segment (start 136.144 42.926) (end 137.70926 44.49126) (width 0.254) (layer B.Cu) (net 12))
 (segment (start 137.70926 44.49126) (end 137.70926 80.53174) (width 0.254) (layer B.Cu) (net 12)))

